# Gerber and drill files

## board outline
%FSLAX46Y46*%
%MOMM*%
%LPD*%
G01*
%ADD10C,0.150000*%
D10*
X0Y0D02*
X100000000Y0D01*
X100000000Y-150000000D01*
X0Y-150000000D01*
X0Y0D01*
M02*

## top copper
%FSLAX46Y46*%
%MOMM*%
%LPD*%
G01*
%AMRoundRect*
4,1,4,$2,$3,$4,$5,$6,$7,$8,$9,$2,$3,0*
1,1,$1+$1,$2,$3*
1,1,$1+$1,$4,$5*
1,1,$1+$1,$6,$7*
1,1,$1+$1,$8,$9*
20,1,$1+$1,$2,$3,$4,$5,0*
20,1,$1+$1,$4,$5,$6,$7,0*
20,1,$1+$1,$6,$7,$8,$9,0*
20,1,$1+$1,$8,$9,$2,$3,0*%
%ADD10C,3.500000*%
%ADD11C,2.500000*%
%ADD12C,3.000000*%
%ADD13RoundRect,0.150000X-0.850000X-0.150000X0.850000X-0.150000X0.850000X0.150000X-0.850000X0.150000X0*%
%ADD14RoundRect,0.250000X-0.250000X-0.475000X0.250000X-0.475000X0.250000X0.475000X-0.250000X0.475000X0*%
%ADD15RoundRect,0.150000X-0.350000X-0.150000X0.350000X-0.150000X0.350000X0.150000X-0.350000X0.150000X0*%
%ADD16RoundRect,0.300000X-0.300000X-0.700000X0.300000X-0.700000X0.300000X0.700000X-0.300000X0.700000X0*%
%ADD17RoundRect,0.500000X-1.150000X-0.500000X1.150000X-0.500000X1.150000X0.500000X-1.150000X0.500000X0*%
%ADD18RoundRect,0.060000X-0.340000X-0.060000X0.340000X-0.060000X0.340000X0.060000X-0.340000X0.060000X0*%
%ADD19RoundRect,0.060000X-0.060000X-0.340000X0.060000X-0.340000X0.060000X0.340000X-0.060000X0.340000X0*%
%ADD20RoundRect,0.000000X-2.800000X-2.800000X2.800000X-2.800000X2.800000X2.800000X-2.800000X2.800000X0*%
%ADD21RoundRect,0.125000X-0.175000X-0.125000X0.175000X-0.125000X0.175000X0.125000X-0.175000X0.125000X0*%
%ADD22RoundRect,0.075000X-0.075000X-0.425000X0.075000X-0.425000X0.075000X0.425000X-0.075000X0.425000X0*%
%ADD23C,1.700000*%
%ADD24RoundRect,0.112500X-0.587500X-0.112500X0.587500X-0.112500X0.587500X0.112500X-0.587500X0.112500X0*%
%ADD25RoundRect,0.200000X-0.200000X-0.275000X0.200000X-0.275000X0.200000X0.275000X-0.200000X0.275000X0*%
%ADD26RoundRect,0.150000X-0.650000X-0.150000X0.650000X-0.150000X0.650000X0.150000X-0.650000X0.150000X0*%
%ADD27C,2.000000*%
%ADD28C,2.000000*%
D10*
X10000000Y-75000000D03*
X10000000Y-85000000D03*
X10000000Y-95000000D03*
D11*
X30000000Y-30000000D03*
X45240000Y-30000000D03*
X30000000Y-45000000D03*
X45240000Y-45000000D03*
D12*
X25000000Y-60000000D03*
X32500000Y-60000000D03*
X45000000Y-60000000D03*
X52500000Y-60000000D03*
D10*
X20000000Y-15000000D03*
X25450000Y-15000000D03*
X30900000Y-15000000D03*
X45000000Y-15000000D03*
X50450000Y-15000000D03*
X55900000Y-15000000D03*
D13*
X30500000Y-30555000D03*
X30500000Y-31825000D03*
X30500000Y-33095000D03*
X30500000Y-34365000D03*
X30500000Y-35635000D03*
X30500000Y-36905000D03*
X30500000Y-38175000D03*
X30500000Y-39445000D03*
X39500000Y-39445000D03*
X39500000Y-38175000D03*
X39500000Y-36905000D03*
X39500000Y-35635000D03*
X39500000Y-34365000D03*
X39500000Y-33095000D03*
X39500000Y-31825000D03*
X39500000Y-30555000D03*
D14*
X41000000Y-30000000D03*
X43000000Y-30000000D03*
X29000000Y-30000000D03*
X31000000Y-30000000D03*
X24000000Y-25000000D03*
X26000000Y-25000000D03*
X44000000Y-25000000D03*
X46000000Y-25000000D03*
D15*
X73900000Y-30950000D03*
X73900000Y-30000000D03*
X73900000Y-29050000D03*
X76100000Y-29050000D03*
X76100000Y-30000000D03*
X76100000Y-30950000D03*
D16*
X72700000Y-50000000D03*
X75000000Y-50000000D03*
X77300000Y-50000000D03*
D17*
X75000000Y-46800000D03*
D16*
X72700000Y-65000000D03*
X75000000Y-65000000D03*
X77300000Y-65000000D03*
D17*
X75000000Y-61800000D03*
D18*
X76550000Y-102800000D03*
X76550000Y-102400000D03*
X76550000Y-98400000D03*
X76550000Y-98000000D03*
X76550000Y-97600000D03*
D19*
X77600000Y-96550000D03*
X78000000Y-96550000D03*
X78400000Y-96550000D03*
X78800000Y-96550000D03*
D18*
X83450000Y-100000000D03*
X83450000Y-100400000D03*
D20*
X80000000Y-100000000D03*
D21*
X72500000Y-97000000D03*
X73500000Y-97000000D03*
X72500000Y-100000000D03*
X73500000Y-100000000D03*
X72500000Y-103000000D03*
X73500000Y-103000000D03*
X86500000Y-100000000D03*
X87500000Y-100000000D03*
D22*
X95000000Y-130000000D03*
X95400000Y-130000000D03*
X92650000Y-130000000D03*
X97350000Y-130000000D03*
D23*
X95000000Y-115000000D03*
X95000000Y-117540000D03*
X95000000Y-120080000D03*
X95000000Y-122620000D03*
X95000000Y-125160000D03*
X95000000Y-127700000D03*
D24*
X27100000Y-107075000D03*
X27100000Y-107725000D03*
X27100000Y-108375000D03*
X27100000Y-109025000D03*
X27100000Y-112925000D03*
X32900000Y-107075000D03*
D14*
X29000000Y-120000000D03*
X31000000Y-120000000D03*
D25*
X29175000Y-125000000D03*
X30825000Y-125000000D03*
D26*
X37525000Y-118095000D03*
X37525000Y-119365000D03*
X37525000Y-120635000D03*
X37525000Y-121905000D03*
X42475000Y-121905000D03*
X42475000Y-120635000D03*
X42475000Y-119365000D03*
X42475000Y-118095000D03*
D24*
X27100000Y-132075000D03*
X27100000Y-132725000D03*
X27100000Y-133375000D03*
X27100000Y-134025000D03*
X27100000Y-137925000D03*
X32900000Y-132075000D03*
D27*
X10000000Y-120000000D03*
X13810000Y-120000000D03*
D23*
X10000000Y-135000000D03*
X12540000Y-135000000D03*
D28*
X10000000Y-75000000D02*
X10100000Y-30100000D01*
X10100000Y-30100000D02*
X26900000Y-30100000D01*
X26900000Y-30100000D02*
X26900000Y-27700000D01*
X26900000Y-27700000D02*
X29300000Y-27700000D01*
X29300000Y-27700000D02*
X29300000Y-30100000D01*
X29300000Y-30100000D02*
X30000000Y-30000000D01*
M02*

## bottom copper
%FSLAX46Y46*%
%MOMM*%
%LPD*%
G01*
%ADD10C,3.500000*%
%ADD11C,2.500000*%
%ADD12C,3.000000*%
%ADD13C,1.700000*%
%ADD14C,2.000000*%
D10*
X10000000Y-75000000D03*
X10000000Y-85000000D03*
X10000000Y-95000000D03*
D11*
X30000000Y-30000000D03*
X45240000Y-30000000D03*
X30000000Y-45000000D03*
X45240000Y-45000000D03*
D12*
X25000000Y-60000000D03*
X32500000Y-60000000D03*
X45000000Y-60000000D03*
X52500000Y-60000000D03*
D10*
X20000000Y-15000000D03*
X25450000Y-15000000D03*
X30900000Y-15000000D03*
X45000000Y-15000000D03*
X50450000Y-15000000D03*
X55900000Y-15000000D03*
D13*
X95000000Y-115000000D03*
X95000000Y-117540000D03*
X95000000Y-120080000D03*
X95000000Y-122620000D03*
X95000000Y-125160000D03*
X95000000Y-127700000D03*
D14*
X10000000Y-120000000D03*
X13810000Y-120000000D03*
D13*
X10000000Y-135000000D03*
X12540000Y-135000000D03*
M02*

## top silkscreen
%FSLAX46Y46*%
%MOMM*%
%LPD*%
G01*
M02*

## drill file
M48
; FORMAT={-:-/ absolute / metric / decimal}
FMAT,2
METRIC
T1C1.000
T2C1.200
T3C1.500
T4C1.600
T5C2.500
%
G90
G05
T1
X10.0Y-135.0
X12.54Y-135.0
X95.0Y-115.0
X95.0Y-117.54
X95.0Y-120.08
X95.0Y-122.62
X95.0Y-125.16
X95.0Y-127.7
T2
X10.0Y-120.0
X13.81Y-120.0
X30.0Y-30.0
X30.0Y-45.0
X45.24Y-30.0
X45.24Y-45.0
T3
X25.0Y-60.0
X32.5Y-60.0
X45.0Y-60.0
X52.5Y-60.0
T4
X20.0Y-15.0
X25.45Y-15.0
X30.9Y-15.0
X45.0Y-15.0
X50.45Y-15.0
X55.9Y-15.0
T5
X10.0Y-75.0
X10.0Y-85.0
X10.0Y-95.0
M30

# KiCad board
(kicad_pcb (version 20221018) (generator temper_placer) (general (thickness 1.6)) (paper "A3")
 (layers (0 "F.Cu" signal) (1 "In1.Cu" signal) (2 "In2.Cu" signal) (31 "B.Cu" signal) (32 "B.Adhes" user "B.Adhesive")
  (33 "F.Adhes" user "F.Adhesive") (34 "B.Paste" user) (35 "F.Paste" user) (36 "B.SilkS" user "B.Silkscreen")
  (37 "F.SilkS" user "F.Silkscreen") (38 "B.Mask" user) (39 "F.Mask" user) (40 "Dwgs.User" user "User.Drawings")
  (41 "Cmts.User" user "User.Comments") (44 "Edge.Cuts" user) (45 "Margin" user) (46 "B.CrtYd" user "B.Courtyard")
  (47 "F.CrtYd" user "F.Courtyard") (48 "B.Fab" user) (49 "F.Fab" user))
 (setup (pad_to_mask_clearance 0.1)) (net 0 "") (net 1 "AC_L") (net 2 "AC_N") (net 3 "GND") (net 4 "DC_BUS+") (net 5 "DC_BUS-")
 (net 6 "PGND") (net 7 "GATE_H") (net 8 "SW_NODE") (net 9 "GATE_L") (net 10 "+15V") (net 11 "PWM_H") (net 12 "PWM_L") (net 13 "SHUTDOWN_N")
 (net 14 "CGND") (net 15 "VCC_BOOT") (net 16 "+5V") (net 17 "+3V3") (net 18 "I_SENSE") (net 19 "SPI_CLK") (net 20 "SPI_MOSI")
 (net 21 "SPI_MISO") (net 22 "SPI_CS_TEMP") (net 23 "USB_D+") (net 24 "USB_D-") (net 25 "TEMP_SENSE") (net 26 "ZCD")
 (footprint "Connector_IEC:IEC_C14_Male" (layer "F.Cu") (at 10 75) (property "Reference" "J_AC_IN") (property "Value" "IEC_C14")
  (pad "1" thru_hole circle (at 0 0) (size 3.5 3.5) (drill 2.5) (layers *.Cu *.Mask) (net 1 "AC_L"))
  (pad "2" thru_hole circle (at 0 10) (size 3.5 3.5) (drill 2.5) (layers *.Cu *.Mask) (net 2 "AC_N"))
  (pad "3" thru_hole circle (at 0 20) (size 3.5 3.5) (drill 2.5) (layers *.Cu *.Mask) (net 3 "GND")))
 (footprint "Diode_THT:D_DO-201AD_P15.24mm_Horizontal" (layer "F.Cu") (at 30 30) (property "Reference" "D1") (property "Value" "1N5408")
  (pad "1" thru_hole circle (at 0 0) (size 2.5 2.5) (drill 1.2) (layers *.Cu *.Mask) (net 1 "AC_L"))
  (pad "2" thru_hole circle (at 15.24 0) (size 2.5 2.5) (drill 1.2) (layers *.Cu *.Mask) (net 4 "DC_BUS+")))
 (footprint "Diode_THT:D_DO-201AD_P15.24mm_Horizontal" (layer "F.Cu") (at 30 45) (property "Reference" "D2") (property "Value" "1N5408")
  (pad "1" thru_hole circle (at 0 0) (size 2.5 2.5) (drill 1.2) (layers *.Cu *.Mask) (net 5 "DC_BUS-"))
  (pad "2" thru_hole circle (at 15.24 0) (size 2.5 2.5) (drill 1.2) (layers *.Cu *.Mask) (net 2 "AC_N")))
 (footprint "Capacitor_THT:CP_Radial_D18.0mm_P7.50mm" (layer "F.Cu") (at 25 60) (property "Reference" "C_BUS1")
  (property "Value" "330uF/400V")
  (pad "1" thru_hole circle (at 0 0) (size 3 3) (drill 1.5) (layers *.Cu *.Mask) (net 4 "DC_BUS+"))
  (pad "2" thru_hole circle (at 7.5 0) (size 3 3) (drill 1.5) (layers *.Cu *.Mask) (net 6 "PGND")))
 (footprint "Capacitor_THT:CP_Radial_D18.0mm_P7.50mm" (layer "F.Cu") (at 45 60) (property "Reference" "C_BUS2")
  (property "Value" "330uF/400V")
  (pad "1" thru_hole circle (at 0 0) (size 3 3) (drill 1.5) (layers *.Cu *.Mask) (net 4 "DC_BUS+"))
  (pad "2" thru_hole circle (at 7.5 0) (size 3 3) (drill 1.5) (layers *.Cu *.Mask) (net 6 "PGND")))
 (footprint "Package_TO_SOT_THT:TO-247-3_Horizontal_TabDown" (layer "F.Cu") (at 20 15) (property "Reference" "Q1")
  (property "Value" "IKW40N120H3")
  (pad "1" thru_hole circle (at 0 0) (size 3.5 3.5) (drill 1.6) (layers *.Cu *.Mask) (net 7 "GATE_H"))
  (pad "2" thru_hole circle (at 5.45 0) (size 3.5 3.5) (drill 1.6) (layers *.Cu *.Mask) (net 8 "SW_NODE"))
  (pad "3" thru_hole circle (at 10.9 0) (size 3.5 3.5) (drill 1.6) (layers *.Cu *.Mask) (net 4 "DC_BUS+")))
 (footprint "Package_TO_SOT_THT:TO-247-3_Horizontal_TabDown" (layer "F.Cu") (at 45 15) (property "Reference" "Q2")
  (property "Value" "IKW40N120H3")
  (pad "1" thru_hole circle (at 0 0) (size 3.5 3.5) (drill 1.6) (layers *.Cu *.Mask) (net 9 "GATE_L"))
  (pad "2" thru_hole circle (at 5.45 0) (size 3.5 3.5) (drill 1.6) (layers *.Cu *.Mask) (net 6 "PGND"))
  (pad "3" thru_hole circle (at 10.9 0) (size 3.5 3.5) (drill 1.6) (layers *.Cu *.Mask) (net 8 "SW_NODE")))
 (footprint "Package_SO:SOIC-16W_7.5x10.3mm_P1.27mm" (layer "F.Cu") (at 35 35) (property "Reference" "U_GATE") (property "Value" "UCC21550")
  (pad "1" smd roundrect (at -4.5 -4.445) (size 2 0.6) (layers "F.Cu" "F.Paste" "F.Mask") (roundrect_rratio 0.25) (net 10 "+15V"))
  (pad "2" smd roundrect (at -4.5 -3.175) (size 2 0.6) (layers "F.Cu" "F.Paste" "F.Mask") (roundrect_rratio 0.25) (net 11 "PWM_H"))
  (pad "3" smd roundrect (at -4.5 -1.905) (size 2 0.6) (layers "F.Cu" "F.Paste" "F.Mask") (roundrect_rratio 0.25) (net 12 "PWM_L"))
  (pad "4" smd roundrect (at -4.5 -0.635) (size 2 0.6) (layers "F.Cu" "F.Paste" "F.Mask") (roundrect_rratio 0.25) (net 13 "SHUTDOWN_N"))
  (pad "5" smd roundrect (at -4.5 0.635) (size 2 0.6) (layers "F.Cu" "F.Paste" "F.Mask") (roundrect_rratio 0.25) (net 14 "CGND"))
  (pad "6" smd roundrect (at -4.5 1.905) (size 2 0.6) (layers "F.Cu" "F.Paste" "F.Mask") (roundrect_rratio 0.25) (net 14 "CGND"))
  (pad "7" smd roundrect (at -4.5 3.175) (size 2 0.6) (layers "F.Cu" "F.Paste" "F.Mask") (roundrect_rratio 0.25) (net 14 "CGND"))
  (pad "8" smd roundrect (at -4.5 4.445) (size 2 0.6) (layers "F.Cu" "F.Paste" "F.Mask") (roundrect_rratio 0.25) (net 14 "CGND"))
  (pad "9" smd roundrect (at 4.5 4.445) (size 2 0.6) (layers "F.Cu" "F.Paste" "F.Mask") (roundrect_rratio 0.25) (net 8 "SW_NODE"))
  (pad "10" smd roundrect (at 4.5 3.175) (size 2 0.6) (layers "F.Cu" "F.Paste" "F.Mask") (roundrect_rratio 0.25) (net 9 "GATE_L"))
  (pad "11" smd roundrect (at 4.5 1.905) (size 2 0.6) (layers "F.Cu" "F.Paste" "F.Mask") (roundrect_rratio 0.25) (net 10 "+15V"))
  (pad "12" smd roundrect (at 4.5 0.635) (size 2 0.6) (layers "F.Cu" "F.Paste" "F.Mask") (roundrect_rratio 0.25) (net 6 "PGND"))
  (pad "13" smd roundrect (at 4.5 -0.635) (size 2 0.6) (layers "F.Cu" "F.Paste" "F.Mask") (roundrect_rratio 0.25) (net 6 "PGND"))
  (pad "14" smd roundrect (at 4.5 -1.905) (size 2 0.6) (layers "F.Cu" "F.Paste" "F.Mask") (roundrect_rratio 0.25) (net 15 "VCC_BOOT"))
  (pad "15" smd roundrect (at 4.5 -3.175) (size 2 0.6) (layers "F.Cu" "F.Paste" "F.Mask") (roundrect_rratio 0.25) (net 7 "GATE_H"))
  (pad "16" smd roundrect (at 4.5 -4.445) (size 2 0.6) (layers "F.Cu" "F.Paste" "F.Mask") (roundrect_rratio 0.25) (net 8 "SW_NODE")))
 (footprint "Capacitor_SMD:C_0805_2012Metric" (layer "F.Cu") (at 42 30) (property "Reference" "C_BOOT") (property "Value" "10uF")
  (pad "1" smd roundrect (at -1 0) (size 1 1.45) (layers "F.Cu" "F.Paste" "F.Mask") (roundrect_rratio 0.25) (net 15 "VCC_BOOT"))
  (pad "2" smd roundrect (at 1 0) (size 1 1.45) (layers "F.Cu" "F.Paste" "F.Mask") (roundrect_rratio 0.25) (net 8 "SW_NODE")))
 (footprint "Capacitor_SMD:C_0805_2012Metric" (layer "F.Cu") (at 30 30) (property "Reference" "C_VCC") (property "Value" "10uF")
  (pad "1" smd roundrect (at -1 0) (size 1 1.45) (layers "F.Cu" "F.Paste" "F.Mask") (roundrect_rratio 0.25) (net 10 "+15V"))
  (pad "2" smd roundrect (at 1 0) (size 1 1.45) (layers "F.Cu" "F.Paste" "F.Mask") (roundrect_rratio 0.25) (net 14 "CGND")))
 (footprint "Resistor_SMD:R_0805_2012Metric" (layer "F.Cu") (at 25 25) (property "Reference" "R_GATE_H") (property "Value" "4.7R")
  (pad "1" smd roundrect (at -1 0) (size 1 1.45) (layers "F.Cu" "F.Paste" "F.Mask") (roundrect_rratio 0.25) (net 7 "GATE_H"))
  (pad "2" smd roundrect (at 1 0) (size 1 1.45) (layers "F.Cu" "F.Paste" "F.Mask") (roundrect_rratio 0.25) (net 7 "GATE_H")))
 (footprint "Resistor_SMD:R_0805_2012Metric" (layer "F.Cu") (at 45 25) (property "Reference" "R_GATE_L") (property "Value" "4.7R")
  (pad "1" smd roundrect (at -1 0) (size 1 1.45) (layers "F.Cu" "F.Paste" "F.Mask") (roundrect_rratio 0.25) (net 9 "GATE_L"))
  (pad "2" smd roundrect (at 1 0) (size 1 1.45) (layers "F.Cu" "F.Paste" "F.Mask") (roundrect_rratio 0.25) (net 9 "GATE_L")))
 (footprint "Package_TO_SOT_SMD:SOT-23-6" (layer "F.Cu") (at 75 30) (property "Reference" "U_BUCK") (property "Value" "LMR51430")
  (pad "1" smd roundrect (at -1.1 0.95) (size 1 0.6) (layers "F.Cu" "F.Paste" "F.Mask") (roundrect_rratio 0.25) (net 3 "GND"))
  (pad "2" smd roundrect (at -1.1 0) (size 1 0.6) (layers "F.Cu" "F.Paste" "F.Mask") (roundrect_rratio 0.25) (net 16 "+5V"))
  (pad "3" smd roundrect (at -1.1 -0.95) (size 1 0.6) (layers "F.Cu" "F.Paste" "F.Mask") (roundrect_rratio 0.25) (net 10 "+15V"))
  (pad "4" smd roundrect (at 1.1 -0.95) (size 1 0.6) (layers "F.Cu" "F.Paste" "F.Mask") (roundrect_rratio 0.25) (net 16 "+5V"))
  (pad "5" smd roundrect (at 1.1 0) (size 1 0.6) (layers "F.Cu" "F.Paste" "F.Mask") (roundrect_rratio 0.25) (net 3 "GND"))
  (pad "6" smd roundrect (at 1.1 0.95) (size 1 0.6) (layers "F.Cu" "F.Paste" "F.Mask") (roundrect_rratio 0.25) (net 3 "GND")))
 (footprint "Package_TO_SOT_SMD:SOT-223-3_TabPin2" (layer "F.Cu") (at 75 50) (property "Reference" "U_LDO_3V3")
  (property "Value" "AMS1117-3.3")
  (pad "1" smd roundrect (at -2.3 0) (size 1.2 2) (layers "F.Cu" "F.Paste" "F.Mask") (roundrect_rratio 0.25) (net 3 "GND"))
  (pad "2" smd roundrect (at 0 0) (size 1.2 2) (layers "F.Cu" "F.Paste" "F.Mask") (roundrect_rratio 0.25) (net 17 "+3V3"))
  (pad "3" smd roundrect (at 2.3 0) (size 1.2 2) (layers "F.Cu" "F.Paste" "F.Mask") (roundrect_rratio 0.25) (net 16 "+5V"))
  (pad "4" smd roundrect (at 0 -3.2) (size 3.3 2) (layers "F.Cu" "F.Paste" "F.Mask") (roundrect_rratio 0.25) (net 17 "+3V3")))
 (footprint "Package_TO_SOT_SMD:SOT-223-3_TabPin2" (layer "F.Cu") (at 75 65) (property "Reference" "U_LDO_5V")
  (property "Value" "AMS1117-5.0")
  (pad "1" smd roundrect (at -2.3 0) (size 1.2 2) (layers "F.Cu" "F.Paste" "F.Mask") (roundrect_rratio 0.25) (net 3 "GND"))
  (pad "2" smd roundrect (at 0 0) (size 1.2 2) (layers "F.Cu" "F.Paste" "F.Mask") (roundrect_rratio 0.25) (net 16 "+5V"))
  (pad "3" smd roundrect (at 2.3 0) (size 1.2 2) (layers "F.Cu" "F.Paste" "F.Mask") (roundrect_rratio 0.25) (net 10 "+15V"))
  (pad "4" smd roundrect (at 0 -3.2) (size 3.3 2) (layers "F.Cu" "F.Paste" "F.Mask") (roundrect_rratio 0.25) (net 16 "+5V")))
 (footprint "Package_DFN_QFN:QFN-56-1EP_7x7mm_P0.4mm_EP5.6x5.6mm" (layer "F.Cu") (at 80 100) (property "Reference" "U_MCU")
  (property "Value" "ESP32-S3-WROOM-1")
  (pad "1" smd roundrect (at -3.45 2.8) (size 0.8 0.24) (layers "F.Cu" "F.Paste" "F.Mask") (roundrect_rratio 0.25) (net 17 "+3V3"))
  (pad "2" smd roundrect (at -3.45 2.4) (size 0.8 0.24) (layers "F.Cu" "F.Paste" "F.Mask") (roundrect_rratio 0.25) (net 3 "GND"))
  (pad "13" smd roundrect (at -3.45 -1.6) (size 0.8 0.24) (layers "F.Cu" "F.Paste" "F.Mask") (roundrect_rratio 0.25) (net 11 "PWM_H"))
  (pad "14" smd roundrect (at -3.45 -2) (size 0.8 0.24) (layers "F.Cu" "F.Paste" "F.Mask") (roundrect_rratio 0.25) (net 12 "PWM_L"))
  (pad "15" smd roundrect (at -3.45 -2.4) (size 0.8 0.24) (layers "F.Cu" "F.Paste" "F.Mask") (roundrect_rratio 0.25) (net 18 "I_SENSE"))
  (pad "20" smd roundrect (at -2.4 -3.45) (size 0.24 0.8) (layers "F.Cu" "F.Paste" "F.Mask") (roundrect_rratio 0.25) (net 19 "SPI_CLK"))
  (pad "21" smd roundrect (at -2 -3.45) (size 0.24 0.8) (layers "F.Cu" "F.Paste" "F.Mask") (roundrect_rratio 0.25) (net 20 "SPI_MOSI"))
  (pad "22" smd roundrect (at -1.6 -3.45) (size 0.24 0.8) (layers "F.Cu" "F.Paste" "F.Mask") (roundrect_rratio 0.25) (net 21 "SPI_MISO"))
  (pad "23" smd roundrect (at -1.2 -3.45) (size 0.24 0.8) (layers "F.Cu" "F.Paste" "F.Mask") (roundrect_rratio 0.25) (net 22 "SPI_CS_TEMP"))
  (pad "40" smd roundrect (at 3.45 0) (size 0.8 0.24) (layers "F.Cu" "F.Paste" "F.Mask") (roundrect_rratio 0.25) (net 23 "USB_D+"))
  (pad "41" smd roundrect (at 3.45 0.4) (size 0.8 0.24) (layers "F.Cu" "F.Paste" "F.Mask") (roundrect_rratio 0.25) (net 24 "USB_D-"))
  (pad "57" smd roundrect (at 0 0) (size 5.6 5.6) (layers "F.Cu" "F.Paste" "F.Mask") (roundrect_rratio 0) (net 3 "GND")))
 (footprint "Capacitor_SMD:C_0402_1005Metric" (layer "F.Cu") (at 73 97) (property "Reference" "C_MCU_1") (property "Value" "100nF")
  (pad "1" smd roundrect (at -0.5 0) (size 0.6 0.5) (layers "F.Cu" "F.Paste" "F.Mask") (roundrect_rratio 0.25) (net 17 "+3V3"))
  (pad "2" smd roundrect (at 0.5 0) (size 0.6 0.5) (layers "F.Cu" "F.Paste" "F.Mask") (roundrect_rratio 0.25) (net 3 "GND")))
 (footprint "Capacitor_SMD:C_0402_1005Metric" (layer "F.Cu") (at 73 100) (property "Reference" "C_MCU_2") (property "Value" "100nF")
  (pad "1" smd roundrect (at -0.5 0) (size 0.6 0.5) (layers "F.Cu" "F.Paste" "F.Mask") (roundrect_rratio 0.25) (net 17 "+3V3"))
  (pad "2" smd roundrect (at 0.5 0) (size 0.6 0.5) (layers "F.Cu" "F.Paste" "F.Mask") (roundrect_rratio 0.25) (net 3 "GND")))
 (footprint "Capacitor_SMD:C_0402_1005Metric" (layer "F.Cu") (at 73 103) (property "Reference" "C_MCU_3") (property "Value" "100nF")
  (pad "1" smd roundrect (at -0.5 0) (size 0.6 0.5) (layers "F.Cu" "F.Paste" "F.Mask") (roundrect_rratio 0.25) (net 17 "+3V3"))
  (pad "2" smd roundrect (at 0.5 0) (size 0.6 0.5) (layers "F.Cu" "F.Paste" "F.Mask") (roundrect_rratio 0.25) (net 3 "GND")))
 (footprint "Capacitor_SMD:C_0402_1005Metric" (layer "F.Cu") (at 87 100) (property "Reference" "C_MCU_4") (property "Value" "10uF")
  (pad "1" smd roundrect (at -0.5 0) (size 0.6 0.5) (layers "F.Cu" "F.Paste" "F.Mask") (roundrect_rratio 0.25) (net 17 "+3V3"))
  (pad "2" smd roundrect (at 0.5 0) (size 0.6 0.5) (layers "F.Cu" "F.Paste" "F.Mask") (roundrect_rratio 0.25) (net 3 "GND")))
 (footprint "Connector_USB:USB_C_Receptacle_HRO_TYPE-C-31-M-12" (layer "F.Cu") (at 95 130) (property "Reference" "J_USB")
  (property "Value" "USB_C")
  (pad "A6" smd roundrect (at 0 0) (size 0.3 1) (layers "F.Cu" "F.Paste" "F.Mask") (roundrect_rratio 0.25) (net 23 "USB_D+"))
  (pad "B6" smd roundrect (at 0.4 0) (size 0.3 1) (layers "F.Cu" "F.Paste" "F.Mask") (roundrect_rratio 0.25) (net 24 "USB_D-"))
  (pad "A1" smd roundrect (at -2.35 0) (size 0.3 1) (layers "F.Cu" "F.Paste" "F.Mask") (roundrect_rratio 0.25) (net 3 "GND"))
  (pad "A12" smd roundrect (at 2.35 0) (size 0.3 1) (layers "F.Cu" "F.Paste" "F.Mask") (roundrect_rratio 0.25) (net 3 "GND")))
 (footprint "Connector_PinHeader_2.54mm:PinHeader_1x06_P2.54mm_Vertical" (layer "F.Cu") (at 95 115) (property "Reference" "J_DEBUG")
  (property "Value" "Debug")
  (pad "1" thru_hole circle (at 0 0) (size 1.7 1.7) (drill 1) (layers *.Cu *.Mask) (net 3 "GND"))
  (pad "2" thru_hole circle (at 0 2.54) (size 1.7 1.7) (drill 1) (layers *.Cu *.Mask) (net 17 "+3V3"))
  (pad "3" thru_hole circle (at 0 5.08) (size 1.7 1.7) (drill 1) (layers *.Cu *.Mask) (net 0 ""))
  (pad "4" thru_hole circle (at 0 7.62) (size 1.7 1.7) (drill 1) (layers *.Cu *.Mask) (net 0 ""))
  (pad "5" thru_hole circle (at 0 10.16) (size 1.7 1.7) (drill 1) (layers *.Cu *.Mask) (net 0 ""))
  (pad "6" thru_hole circle (at 0 12.7) (size 1.7 1.7) (drill 1) (layers *.Cu *.Mask) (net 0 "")))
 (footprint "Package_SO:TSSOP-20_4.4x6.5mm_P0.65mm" (layer "F.Cu") (at 30 110) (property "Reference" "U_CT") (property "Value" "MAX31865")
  (pad "1" smd roundrect (at -2.9 -2.925) (size 1.4 0.45) (layers "F.Cu" "F.Paste" "F.Mask") (roundrect_rratio 0.25) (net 19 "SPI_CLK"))
  (pad "2" smd roundrect (at -2.9 -2.275) (size 1.4 0.45) (layers "F.Cu" "F.Paste" "F.Mask") (roundrect_rratio 0.25) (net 20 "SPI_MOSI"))
  (pad "3" smd roundrect (at -2.9 -1.625) (size 1.4 0.45) (layers "F.Cu" "F.Paste" "F.Mask") (roundrect_rratio 0.25) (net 21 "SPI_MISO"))
  (pad "4" smd roundrect (at -2.9 -0.975) (size 1.4 0.45) (layers "F.Cu" "F.Paste" "F.Mask") (roundrect_rratio 0.25) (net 22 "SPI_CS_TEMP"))
  (pad "10" smd roundrect (at -2.9 2.925) (size 1.4 0.45) (layers "F.Cu" "F.Paste" "F.Mask") (roundrect_rratio 0.25) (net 3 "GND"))
  (pad "20" smd roundrect (at 2.9 -2.925) (size 1.4 0.45) (layers "F.Cu" "F.Paste" "F.Mask") (roundrect_rratio 0.25) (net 17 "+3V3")))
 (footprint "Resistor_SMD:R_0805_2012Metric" (layer "F.Cu") (at 30 120) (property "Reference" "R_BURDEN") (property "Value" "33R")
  (pad "1" smd roundrect (at -1 0) (size 1 1.45) (layers "F.Cu" "F.Paste" "F.Mask") (roundrect_rratio 0.25) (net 18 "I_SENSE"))
  (pad "2" smd roundrect (at 1 0) (size 1 1.45) (layers "F.Cu" "F.Paste" "F.Mask") (roundrect_rratio 0.25) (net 3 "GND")))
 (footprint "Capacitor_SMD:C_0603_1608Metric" (layer "F.Cu") (at 30 125) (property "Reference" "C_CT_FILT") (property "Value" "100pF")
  (pad "1" smd roundrect (at -0.825 0) (size 0.8 0.95) (layers "F.Cu" "F.Paste" "F.Mask") (roundrect_rratio 0.25) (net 18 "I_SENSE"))
  (pad "2" smd roundrect (at 0.825 0) (size 0.8 0.95) (layers "F.Cu" "F.Paste" "F.Mask") (roundrect_rratio 0.25) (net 3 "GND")))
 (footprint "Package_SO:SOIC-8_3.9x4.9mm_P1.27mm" (layer "F.Cu") (at 40 120) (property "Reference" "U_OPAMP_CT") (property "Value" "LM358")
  (pad "1" smd roundrect (at -2.475 -1.905) (size 1.6 0.6) (layers "F.Cu" "F.Paste" "F.Mask") (roundrect_rratio 0.25) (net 18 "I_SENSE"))
  (pad "2" smd roundrect (at -2.475 -0.635) (size 1.6 0.6) (layers "F.Cu" "F.Paste" "F.Mask") (roundrect_rratio 0.25) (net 18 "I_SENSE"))
  (pad "3" smd roundrect (at -2.475 0.635) (size 1.6 0.6) (layers "F.Cu" "F.Paste" "F.Mask") (roundrect_rratio 0.25) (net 18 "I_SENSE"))
  (pad "4" smd roundrect (at -2.475 1.905) (size 1.6 0.6) (layers "F.Cu" "F.Paste" "F.Mask") (roundrect_rratio 0.25) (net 3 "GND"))
  (pad "5" smd roundrect (at 2.475 1.905) (size 1.6 0.6) (layers "F.Cu" "F.Paste" "F.Mask") (roundrect_rratio 0.25) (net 18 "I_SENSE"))
  (pad "6" smd roundrect (at 2.475 0.635) (size 1.6 0.6) (layers "F.Cu" "F.Paste" "F.Mask") (roundrect_rratio 0.25) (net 18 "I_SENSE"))
  (pad "7" smd roundrect (at 2.475 -0.635) (size 1.6 0.6) (layers "F.Cu" "F.Paste" "F.Mask") (roundrect_rratio 0.25) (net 16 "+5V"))
  (pad "8" smd roundrect (at 2.475 -1.905) (size 1.6 0.6) (layers "F.Cu" "F.Paste" "F.Mask") (roundrect_rratio 0.25) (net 16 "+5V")))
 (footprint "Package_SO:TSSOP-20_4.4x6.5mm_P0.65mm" (layer "F.Cu") (at 30 135) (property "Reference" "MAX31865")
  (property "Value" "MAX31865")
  (pad "1" smd roundrect (at -2.9 -2.925) (size 1.4 0.45) (layers "F.Cu" "F.Paste" "F.Mask") (roundrect_rratio 0.25) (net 19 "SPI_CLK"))
  (pad "2" smd roundrect (at -2.9 -2.275) (size 1.4 0.45) (layers "F.Cu" "F.Paste" "F.Mask") (roundrect_rratio 0.25) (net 20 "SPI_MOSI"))
  (pad "3" smd roundrect (at -2.9 -1.625) (size 1.4 0.45) (layers "F.Cu" "F.Paste" "F.Mask") (roundrect_rratio 0.25) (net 21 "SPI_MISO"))
  (pad "4" smd roundrect (at -2.9 -0.975) (size 1.4 0.45) (layers "F.Cu" "F.Paste" "F.Mask") (roundrect_rratio 0.25) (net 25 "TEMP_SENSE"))
  (pad "10" smd roundrect (at -2.9 2.925) (size 1.4 0.45) (layers "F.Cu" "F.Paste" "F.Mask") (roundrect_rratio 0.25) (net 3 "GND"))
  (pad "20" smd roundrect (at 2.9 -2.925) (size 1.4 0.45) (layers "F.Cu" "F.Paste" "F.Mask") (roundrect_rratio 0.25) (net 17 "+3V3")))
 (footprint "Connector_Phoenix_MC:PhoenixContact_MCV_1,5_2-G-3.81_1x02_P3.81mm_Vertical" (layer "F.Cu") (at 10 120)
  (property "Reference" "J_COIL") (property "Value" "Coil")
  (pad "1" thru_hole circle (at 0 0) (size 2 2) (drill 1.2) (layers *.Cu *.Mask) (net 8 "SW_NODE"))
  (pad "2" thru_hole circle (at 3.81 0) (size 2 2) (drill 1.2) (layers *.Cu *.Mask) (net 3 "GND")))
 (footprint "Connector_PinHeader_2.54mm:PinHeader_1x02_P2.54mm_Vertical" (layer "F.Cu") (at 10 135) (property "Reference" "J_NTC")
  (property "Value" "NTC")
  (pad "1" thru_hole circle (at 0 0) (size 1.7 1.7) (drill 1) (layers *.Cu *.Mask) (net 25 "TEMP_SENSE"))
  (pad "2" thru_hole circle (at 2.54 0) (size 1.7 1.7) (drill 1) (layers *.Cu *.Mask) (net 3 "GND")))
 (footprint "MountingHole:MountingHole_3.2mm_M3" (layer "F.Cu") (at 5 5) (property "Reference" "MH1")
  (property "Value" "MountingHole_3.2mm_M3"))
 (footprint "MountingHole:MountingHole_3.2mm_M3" (layer "F.Cu") (at 95 5) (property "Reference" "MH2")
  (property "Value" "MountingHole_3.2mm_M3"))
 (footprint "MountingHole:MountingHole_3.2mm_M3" (layer "F.Cu") (at 5 145) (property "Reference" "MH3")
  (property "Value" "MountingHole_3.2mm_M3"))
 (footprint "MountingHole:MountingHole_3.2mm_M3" (layer "F.Cu") (at 95 145) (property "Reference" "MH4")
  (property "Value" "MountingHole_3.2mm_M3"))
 (gr_rect (start 0 0) (end 100 150) (layer "Edge.Cuts") (width 0.15))
 (segment (start 10.0 75.0) (end 10.1 30.1) (width 2.0) (layer "F.Cu") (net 1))
 (segment (start 10.1 30.1) (end 26.900000000000002 30.1) (width 2.0) (layer "F.Cu") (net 1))
 (segment (start 26.900000000000002 30.1) (end 26.900000000000002 27.700000000000003) (width 2.0) (layer "F.Cu") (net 1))
 (segment (start 26.900000000000002 27.700000000000003) (end 29.300000000000004 27.700000000000003) (width 2.0) (layer "F.Cu") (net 1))
 (segment (start 29.300000000000004 27.700000000000003) (end 29.300000000000004 30.1) (width 2.0) (layer "F.Cu") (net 1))
 (segment (start 29.300000000000004 30.1) (end 30.0 30.0) (width 2.0) (layer "F.Cu") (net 1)))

